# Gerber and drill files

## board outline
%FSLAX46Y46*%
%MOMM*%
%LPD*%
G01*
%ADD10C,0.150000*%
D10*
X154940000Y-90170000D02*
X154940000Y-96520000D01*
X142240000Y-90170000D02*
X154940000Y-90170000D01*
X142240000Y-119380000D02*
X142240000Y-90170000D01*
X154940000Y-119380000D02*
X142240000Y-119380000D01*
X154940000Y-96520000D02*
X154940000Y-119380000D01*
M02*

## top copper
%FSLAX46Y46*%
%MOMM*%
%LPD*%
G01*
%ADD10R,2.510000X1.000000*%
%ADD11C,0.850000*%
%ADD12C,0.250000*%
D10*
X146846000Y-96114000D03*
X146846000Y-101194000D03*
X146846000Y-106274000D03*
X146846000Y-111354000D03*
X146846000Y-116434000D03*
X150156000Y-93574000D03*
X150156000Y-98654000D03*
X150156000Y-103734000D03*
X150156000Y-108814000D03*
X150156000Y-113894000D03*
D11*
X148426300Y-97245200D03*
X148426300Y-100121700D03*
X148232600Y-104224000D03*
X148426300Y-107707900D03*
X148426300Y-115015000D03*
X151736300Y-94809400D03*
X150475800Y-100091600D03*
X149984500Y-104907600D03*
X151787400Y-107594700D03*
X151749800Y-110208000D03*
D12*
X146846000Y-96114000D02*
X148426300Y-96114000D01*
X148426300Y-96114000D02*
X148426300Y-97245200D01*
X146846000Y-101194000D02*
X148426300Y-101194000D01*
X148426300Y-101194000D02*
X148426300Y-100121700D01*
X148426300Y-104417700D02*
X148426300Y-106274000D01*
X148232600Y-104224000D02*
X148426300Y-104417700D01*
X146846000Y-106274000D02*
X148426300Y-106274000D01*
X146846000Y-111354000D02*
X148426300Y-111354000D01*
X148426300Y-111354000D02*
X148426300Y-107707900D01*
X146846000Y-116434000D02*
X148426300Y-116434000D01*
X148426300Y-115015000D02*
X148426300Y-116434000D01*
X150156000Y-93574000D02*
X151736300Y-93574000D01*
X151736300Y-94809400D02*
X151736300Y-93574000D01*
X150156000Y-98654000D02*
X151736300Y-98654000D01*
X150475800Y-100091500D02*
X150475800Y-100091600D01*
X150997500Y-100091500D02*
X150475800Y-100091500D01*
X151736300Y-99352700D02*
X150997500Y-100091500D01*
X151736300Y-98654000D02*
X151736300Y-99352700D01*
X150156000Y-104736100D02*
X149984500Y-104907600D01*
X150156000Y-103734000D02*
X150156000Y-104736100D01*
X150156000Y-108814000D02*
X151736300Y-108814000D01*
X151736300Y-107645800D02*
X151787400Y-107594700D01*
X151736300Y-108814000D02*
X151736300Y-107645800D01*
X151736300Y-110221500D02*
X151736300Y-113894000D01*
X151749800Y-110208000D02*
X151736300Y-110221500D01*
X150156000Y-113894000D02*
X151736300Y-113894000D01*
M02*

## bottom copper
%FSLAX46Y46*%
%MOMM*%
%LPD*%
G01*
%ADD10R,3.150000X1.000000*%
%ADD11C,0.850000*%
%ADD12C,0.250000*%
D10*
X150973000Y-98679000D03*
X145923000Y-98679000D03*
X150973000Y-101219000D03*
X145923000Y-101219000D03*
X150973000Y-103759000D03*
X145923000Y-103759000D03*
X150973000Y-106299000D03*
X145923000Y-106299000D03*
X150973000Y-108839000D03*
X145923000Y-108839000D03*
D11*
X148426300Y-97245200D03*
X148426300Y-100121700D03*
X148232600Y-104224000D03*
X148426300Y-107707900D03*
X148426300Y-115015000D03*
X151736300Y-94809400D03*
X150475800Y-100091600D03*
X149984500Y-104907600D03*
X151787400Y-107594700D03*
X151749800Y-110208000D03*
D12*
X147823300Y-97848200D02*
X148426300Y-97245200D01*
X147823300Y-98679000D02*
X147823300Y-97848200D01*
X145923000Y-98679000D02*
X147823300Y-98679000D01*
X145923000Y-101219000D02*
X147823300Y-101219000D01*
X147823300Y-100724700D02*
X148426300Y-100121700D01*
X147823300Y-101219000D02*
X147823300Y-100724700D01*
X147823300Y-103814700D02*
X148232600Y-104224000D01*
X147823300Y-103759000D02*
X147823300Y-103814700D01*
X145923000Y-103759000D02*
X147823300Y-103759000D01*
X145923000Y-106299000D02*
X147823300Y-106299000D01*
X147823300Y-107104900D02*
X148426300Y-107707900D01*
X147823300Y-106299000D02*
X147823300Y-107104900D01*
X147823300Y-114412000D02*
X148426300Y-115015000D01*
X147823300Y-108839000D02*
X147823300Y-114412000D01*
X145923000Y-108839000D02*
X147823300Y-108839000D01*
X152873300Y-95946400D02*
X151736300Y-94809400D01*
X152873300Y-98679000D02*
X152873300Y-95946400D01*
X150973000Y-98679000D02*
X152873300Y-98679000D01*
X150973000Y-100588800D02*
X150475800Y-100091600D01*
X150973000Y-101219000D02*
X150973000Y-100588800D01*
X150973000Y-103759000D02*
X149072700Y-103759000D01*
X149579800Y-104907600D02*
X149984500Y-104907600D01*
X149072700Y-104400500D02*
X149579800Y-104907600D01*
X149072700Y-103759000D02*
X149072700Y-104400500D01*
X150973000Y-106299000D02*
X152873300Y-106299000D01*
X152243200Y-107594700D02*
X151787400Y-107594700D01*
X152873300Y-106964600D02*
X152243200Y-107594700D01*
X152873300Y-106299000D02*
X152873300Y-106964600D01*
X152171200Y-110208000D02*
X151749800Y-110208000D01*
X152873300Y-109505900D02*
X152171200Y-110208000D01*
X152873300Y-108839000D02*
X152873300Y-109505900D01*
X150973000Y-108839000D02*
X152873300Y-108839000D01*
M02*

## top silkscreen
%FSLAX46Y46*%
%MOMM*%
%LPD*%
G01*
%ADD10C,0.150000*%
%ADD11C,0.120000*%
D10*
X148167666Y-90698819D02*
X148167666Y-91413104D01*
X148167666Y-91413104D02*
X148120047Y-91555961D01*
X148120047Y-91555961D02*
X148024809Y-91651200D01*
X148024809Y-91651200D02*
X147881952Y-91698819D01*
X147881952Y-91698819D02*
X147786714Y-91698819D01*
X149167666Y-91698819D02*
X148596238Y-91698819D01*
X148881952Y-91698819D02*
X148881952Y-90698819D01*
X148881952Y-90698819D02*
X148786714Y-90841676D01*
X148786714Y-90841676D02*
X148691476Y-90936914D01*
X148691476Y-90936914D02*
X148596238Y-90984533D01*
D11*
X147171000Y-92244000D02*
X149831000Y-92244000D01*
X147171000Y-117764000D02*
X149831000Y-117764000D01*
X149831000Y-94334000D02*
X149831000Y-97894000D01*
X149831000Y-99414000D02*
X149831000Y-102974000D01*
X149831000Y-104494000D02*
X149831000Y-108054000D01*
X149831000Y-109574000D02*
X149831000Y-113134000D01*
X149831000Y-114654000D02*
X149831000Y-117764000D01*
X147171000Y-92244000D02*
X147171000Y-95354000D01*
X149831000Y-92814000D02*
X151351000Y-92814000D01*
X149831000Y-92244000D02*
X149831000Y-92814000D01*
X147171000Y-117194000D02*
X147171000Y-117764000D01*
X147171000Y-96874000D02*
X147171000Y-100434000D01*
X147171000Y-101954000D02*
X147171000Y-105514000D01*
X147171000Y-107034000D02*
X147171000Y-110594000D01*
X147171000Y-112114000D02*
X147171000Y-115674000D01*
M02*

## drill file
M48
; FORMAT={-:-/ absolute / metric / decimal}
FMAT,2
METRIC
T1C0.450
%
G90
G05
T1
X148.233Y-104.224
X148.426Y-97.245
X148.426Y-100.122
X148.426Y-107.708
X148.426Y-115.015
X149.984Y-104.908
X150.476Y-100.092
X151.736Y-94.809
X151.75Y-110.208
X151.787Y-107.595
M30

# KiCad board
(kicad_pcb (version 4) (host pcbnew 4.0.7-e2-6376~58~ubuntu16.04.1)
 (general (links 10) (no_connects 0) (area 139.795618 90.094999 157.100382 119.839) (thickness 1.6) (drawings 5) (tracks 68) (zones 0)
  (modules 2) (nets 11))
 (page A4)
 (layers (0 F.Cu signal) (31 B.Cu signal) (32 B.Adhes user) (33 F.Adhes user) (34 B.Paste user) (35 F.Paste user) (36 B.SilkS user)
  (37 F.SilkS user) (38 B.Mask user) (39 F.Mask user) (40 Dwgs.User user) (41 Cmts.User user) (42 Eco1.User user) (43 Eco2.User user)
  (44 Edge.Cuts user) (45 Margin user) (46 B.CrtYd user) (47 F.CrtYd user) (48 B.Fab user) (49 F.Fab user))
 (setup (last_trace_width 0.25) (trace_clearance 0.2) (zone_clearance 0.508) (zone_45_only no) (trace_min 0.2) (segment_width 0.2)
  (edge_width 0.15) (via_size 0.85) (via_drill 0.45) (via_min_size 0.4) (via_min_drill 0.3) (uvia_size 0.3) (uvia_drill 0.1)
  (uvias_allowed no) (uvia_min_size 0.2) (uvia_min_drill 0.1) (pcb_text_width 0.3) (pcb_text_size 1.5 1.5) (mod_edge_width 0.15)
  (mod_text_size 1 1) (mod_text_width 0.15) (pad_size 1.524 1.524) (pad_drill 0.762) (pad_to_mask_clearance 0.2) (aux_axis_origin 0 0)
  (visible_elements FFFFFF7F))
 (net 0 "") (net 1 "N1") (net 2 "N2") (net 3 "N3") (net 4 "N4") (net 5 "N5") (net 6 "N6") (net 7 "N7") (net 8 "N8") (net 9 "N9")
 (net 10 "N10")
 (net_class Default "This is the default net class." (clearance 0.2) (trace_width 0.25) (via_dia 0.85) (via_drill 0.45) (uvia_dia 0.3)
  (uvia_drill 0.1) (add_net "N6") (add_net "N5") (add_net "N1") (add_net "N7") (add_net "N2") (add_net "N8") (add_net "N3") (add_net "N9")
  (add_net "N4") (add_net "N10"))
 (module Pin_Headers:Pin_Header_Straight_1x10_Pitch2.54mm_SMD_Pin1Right (layer F.Cu) (at 148.501 105.004)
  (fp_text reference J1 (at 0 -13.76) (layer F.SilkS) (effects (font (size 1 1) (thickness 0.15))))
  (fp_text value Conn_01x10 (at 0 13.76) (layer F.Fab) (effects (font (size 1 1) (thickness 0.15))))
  (fp_line (start -1.33 -12.76) (end 1.33 -12.76) (layer F.SilkS) (width 0.12))
  (fp_line (start -1.33 12.76) (end 1.33 12.76) (layer F.SilkS) (width 0.12))
  (fp_line (start 1.33 -10.67) (end 1.33 -7.11) (layer F.SilkS) (width 0.12))
  (fp_line (start 1.33 -5.59) (end 1.33 -2.03) (layer F.SilkS) (width 0.12))
  (fp_line (start 1.33 -0.51) (end 1.33 3.05) (layer F.SilkS) (width 0.12))
  (fp_line (start 1.33 4.57) (end 1.33 8.13) (layer F.SilkS) (width 0.12))
  (fp_line (start 1.33 9.65) (end 1.33 12.76) (layer F.SilkS) (width 0.12))
  (fp_line (start -1.33 -12.76) (end -1.33 -9.65) (layer F.SilkS) (width 0.12))
  (fp_line (start 1.33 -12.19) (end 2.85 -12.19) (layer F.SilkS) (width 0.12))
  (fp_line (start 1.33 -12.76) (end 1.33 -12.19) (layer F.SilkS) (width 0.12))
  (fp_line (start -1.33 12.19) (end -1.33 12.76) (layer F.SilkS) (width 0.12))
  (fp_line (start -1.33 -8.13) (end -1.33 -4.57) (layer F.SilkS) (width 0.12))
  (fp_line (start -1.33 -3.05) (end -1.33 0.51) (layer F.SilkS) (width 0.12))
  (fp_line (start -1.33 2.03) (end -1.33 5.59) (layer F.SilkS) (width 0.12))
  (fp_line (start -1.33 7.11) (end -1.33 10.67) (layer F.SilkS) (width 0.12))
  (pad 2 smd rect (at -1.655 -8.89) (size 2.51 1) (layers F.Cu F.Paste F.Mask) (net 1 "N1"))
  (pad 4 smd rect (at -1.655 -3.81) (size 2.51 1) (layers F.Cu F.Paste F.Mask) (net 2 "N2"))
  (pad 6 smd rect (at -1.655 1.27) (size 2.51 1) (layers F.Cu F.Paste F.Mask) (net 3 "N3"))
  (pad 8 smd rect (at -1.655 6.35) (size 2.51 1) (layers F.Cu F.Paste F.Mask) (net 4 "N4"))
  (pad 10 smd rect (at -1.655 11.43) (size 2.51 1) (layers F.Cu F.Paste F.Mask) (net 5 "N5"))
  (pad 1 smd rect (at 1.655 -11.43) (size 2.51 1) (layers F.Cu F.Paste F.Mask) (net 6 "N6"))
  (pad 3 smd rect (at 1.655 -6.35) (size 2.51 1) (layers F.Cu F.Paste F.Mask) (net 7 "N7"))
  (pad 5 smd rect (at 1.655 -1.27) (size 2.51 1) (layers F.Cu F.Paste F.Mask) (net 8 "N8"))
  (pad 7 smd rect (at 1.655 3.81) (size 2.51 1) (layers F.Cu F.Paste F.Mask) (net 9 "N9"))
  (pad 9 smd rect (at 1.655 8.89) (size 2.51 1) (layers F.Cu F.Paste F.Mask) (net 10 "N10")))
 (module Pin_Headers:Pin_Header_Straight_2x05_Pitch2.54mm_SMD (layer B.Cu) (at 148.448 103.759 180)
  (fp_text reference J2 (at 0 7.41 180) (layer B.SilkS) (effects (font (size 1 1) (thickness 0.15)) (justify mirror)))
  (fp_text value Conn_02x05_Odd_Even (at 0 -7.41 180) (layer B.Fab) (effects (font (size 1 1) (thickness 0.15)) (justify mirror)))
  (pad 1 smd rect (at -2.525 5.08 180) (size 3.15 1) (layers B.Cu B.Paste B.Mask) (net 6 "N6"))
  (pad 2 smd rect (at 2.525 5.08 180) (size 3.15 1) (layers B.Cu B.Paste B.Mask) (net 1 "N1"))
  (pad 3 smd rect (at -2.525 2.54 180) (size 3.15 1) (layers B.Cu B.Paste B.Mask) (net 7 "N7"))
  (pad 4 smd rect (at 2.525 2.54 180) (size 3.15 1) (layers B.Cu B.Paste B.Mask) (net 2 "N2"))
  (pad 5 smd rect (at -2.525 0 180) (size 3.15 1) (layers B.Cu B.Paste B.Mask) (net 8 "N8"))
  (pad 6 smd rect (at 2.525 0 180) (size 3.15 1) (layers B.Cu B.Paste B.Mask) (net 3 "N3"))
  (pad 7 smd rect (at -2.525 -2.54 180) (size 3.15 1) (layers B.Cu B.Paste B.Mask) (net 9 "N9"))
  (pad 8 smd rect (at 2.525 -2.54 180) (size 3.15 1) (layers B.Cu B.Paste B.Mask) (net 4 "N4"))
  (pad 9 smd rect (at -2.525 -5.08 180) (size 3.15 1) (layers B.Cu B.Paste B.Mask) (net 10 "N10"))
  (pad 10 smd rect (at 2.525 -5.08 180) (size 3.15 1) (layers B.Cu B.Paste B.Mask) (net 5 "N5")))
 (gr_line (start 154.94 90.17) (end 154.94 96.52) (layer Edge.Cuts) (width 0.15))
 (gr_line (start 142.24 90.17) (end 154.94 90.17) (layer Edge.Cuts) (width 0.15))
 (gr_line (start 142.24 119.38) (end 142.24 90.17) (layer Edge.Cuts) (width 0.15))
 (gr_line (start 154.94 119.38) (end 142.24 119.38) (layer Edge.Cuts) (width 0.15))
 (gr_line (start 154.94 96.52) (end 154.94 119.38) (layer Edge.Cuts) (width 0.15))
 (via (at 148.4263 97.2452) (size 0.85) (layers F.Cu B.Cu) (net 1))
 (segment (start 146.846 96.114) (end 148.4263 96.114) (width 0.25) (layer F.Cu) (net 1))
 (segment (start 147.8233 97.8482) (end 148.4263 97.2452) (width 0.25) (layer B.Cu) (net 1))
 (segment (start 147.8233 98.679) (end 147.8233 97.8482) (width 0.25) (layer B.Cu) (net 1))
 (segment (start 148.4263 96.114) (end 148.4263 97.2452) (width 0.25) (layer F.Cu) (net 1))
 (segment (start 145.923 98.679) (end 147.8233 98.679) (width 0.25) (layer B.Cu) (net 1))
 (via (at 148.4263 100.1217) (size 0.85) (layers F.Cu B.Cu) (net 2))
 (segment (start 146.846 101.194) (end 148.4263 101.194) (width 0.25) (layer F.Cu) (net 2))
 (segment (start 145.923 101.219) (end 147.8233 101.219) (width 0.25) (layer B.Cu) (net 2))
 (segment (start 147.8233 100.7247) (end 148.4263 100.1217) (width 0.25) (layer B.Cu) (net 2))
 (segment (start 147.8233 101.219) (end 147.8233 100.7247) (width 0.25) (layer B.Cu) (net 2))
 (segment (start 148.4263 101.194) (end 148.4263 100.1217) (width 0.25) (layer F.Cu) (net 2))
 (via (at 148.2326 104.224) (size 0.85) (layers F.Cu B.Cu) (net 3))
 (segment (start 147.8233 103.8147) (end 148.2326 104.224) (width 0.25) (layer B.Cu) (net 3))
 (segment (start 147.8233 103.759) (end 147.8233 103.8147) (width 0.25) (layer B.Cu) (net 3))
 (segment (start 148.4263 104.4177) (end 148.4263 106.274) (width 0.25) (layer F.Cu) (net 3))
 (segment (start 148.2326 104.224) (end 148.4263 104.4177) (width 0.25) (layer F.Cu) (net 3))
 (segment (start 146.846 106.274) (end 148.4263 106.274) (width 0.25) (layer F.Cu) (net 3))
 (segment (start 145.923 103.759) (end 147.8233 103.759) (width 0.25) (layer B.Cu) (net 3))
 (via (at 148.4263 107.7079) (size 0.85) (layers F.Cu B.Cu) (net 4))
 (segment (start 146.846 111.354) (end 148.4263 111.354) (width 0.25) (layer F.Cu) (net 4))
 (segment (start 145.923 106.299) (end 147.8233 106.299) (width 0.25) (layer B.Cu) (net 4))
 (segment (start 147.8233 107.1049) (end 148.4263 107.7079) (width 0.25) (layer B.Cu) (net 4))
 (segment (start 147.8233 106.299) (end 147.8233 107.1049) (width 0.25) (layer B.Cu) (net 4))
 (segment (start 148.4263 111.354) (end 148.4263 107.7079) (width 0.25) (layer F.Cu) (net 4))
 (via (at 148.4263 115.015) (size 0.85) (layers F.Cu B.Cu) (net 5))
 (segment (start 146.846 116.434) (end 148.4263 116.434) (width 0.25) (layer F.Cu) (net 5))
 (segment (start 147.8233 114.412) (end 148.4263 115.015) (width 0.25) (layer B.Cu) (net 5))
 (segment (start 147.8233 108.839) (end 147.8233 114.412) (width 0.25) (layer B.Cu) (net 5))
 (segment (start 148.4263 115.015) (end 148.4263 116.434) (width 0.25) (layer F.Cu) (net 5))
 (segment (start 145.923 108.839) (end 147.8233 108.839) (width 0.25) (layer B.Cu) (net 5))
 (via (at 151.7363 94.8094) (size 0.85) (layers F.Cu B.Cu) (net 6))
 (segment (start 150.156 93.574) (end 151.7363 93.574) (width 0.25) (layer F.Cu) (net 6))
 (segment (start 152.8733 95.9464) (end 151.7363 94.8094) (width 0.25) (layer B.Cu) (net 6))
 (segment (start 152.8733 98.679) (end 152.8733 95.9464) (width 0.25) (layer B.Cu) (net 6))
 (segment (start 151.7363 94.8094) (end 151.7363 93.574) (width 0.25) (layer F.Cu) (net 6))
 (segment (start 150.973 98.679) (end 152.8733 98.679) (width 0.25) (layer B.Cu) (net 6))
 (via (at 150.4758 100.0916) (size 0.85) (layers F.Cu B.Cu) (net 7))
 (segment (start 150.156 98.654) (end 151.7363 98.654) (width 0.25) (layer F.Cu) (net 7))
 (segment (start 150.973 100.5888) (end 150.4758 100.0916) (width 0.25) (layer B.Cu) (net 7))
 (segment (start 150.973 101.219) (end 150.973 100.5888) (width 0.25) (layer B.Cu) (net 7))
 (segment (start 150.4758 100.0915) (end 150.4758 100.0916) (width 0.25) (layer F.Cu) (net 7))
 (segment (start 150.9975 100.0915) (end 150.4758 100.0915) (width 0.25) (layer F.Cu) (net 7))
 (segment (start 151.7363 99.3527) (end 150.9975 100.0915) (width 0.25) (layer F.Cu) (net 7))
 (segment (start 151.7363 98.654) (end 151.7363 99.3527) (width 0.25) (layer F.Cu) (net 7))
 (via (at 149.9845 104.9076) (size 0.85) (layers F.Cu B.Cu) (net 8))
 (segment (start 150.973 103.759) (end 149.0727 103.759) (width 0.25) (layer B.Cu) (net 8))
 (segment (start 149.5798 104.9076) (end 149.9845 104.9076) (width 0.25) (layer B.Cu) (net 8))
 (segment (start 149.0727 104.4005) (end 149.5798 104.9076) (width 0.25) (layer B.Cu) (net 8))
 (segment (start 149.0727 103.759) (end 149.0727 104.4005) (width 0.25) (layer B.Cu) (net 8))
 (segment (start 150.156 104.7361) (end 149.9845 104.9076) (width 0.25) (layer F.Cu) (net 8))
 (segment (start 150.156 103.734) (end 150.156 104.7361) (width 0.25) (layer F.Cu) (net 8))
 (via (at 151.7874 107.5947) (size 0.85) (layers F.Cu B.Cu) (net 9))
 (segment (start 150.156 108.814) (end 151.7363 108.814) (width 0.25) (layer F.Cu) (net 9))
 (segment (start 150.973 106.299) (end 152.8733 106.299) (width 0.25) (layer B.Cu) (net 9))
 (segment (start 152.2432 107.5947) (end 151.7874 107.5947) (width 0.25) (layer B.Cu) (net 9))
 (segment (start 152.8733 106.9646) (end 152.2432 107.5947) (width 0.25) (layer B.Cu) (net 9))
 (segment (start 152.8733 106.299) (end 152.8733 106.9646) (width 0.25) (layer B.Cu) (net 9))
 (segment (start 151.7363 107.6458) (end 151.7874 107.5947) (width 0.25) (layer F.Cu) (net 9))
 (segment (start 151.7363 108.814) (end 151.7363 107.6458) (width 0.25) (layer F.Cu) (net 9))
 (via (at 151.7498 110.208) (size 0.85) (layers F.Cu B.Cu) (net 10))
 (segment (start 152.1712 110.208) (end 151.7498 110.208) (width 0.25) (layer B.Cu) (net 10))
 (segment (start 152.8733 109.5059) (end 152.1712 110.208) (width 0.25) (layer B.Cu) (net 10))
 (segment (start 152.8733 108.839) (end 152.8733 109.5059) (width 0.25) (layer B.Cu) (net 10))
 (segment (start 151.7363 110.2215) (end 151.7363 113.894) (width 0.25) (layer F.Cu) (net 10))
 (segment (start 151.7498 110.208) (end 151.7363 110.2215) (width 0.25) (layer F.Cu) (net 10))
 (segment (start 150.156 113.894) (end 151.7363 113.894) (width 0.25) (layer F.Cu) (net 10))
 (segment (start 150.973 108.839) (end 152.8733 108.839) (width 0.25) (layer B.Cu) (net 10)))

